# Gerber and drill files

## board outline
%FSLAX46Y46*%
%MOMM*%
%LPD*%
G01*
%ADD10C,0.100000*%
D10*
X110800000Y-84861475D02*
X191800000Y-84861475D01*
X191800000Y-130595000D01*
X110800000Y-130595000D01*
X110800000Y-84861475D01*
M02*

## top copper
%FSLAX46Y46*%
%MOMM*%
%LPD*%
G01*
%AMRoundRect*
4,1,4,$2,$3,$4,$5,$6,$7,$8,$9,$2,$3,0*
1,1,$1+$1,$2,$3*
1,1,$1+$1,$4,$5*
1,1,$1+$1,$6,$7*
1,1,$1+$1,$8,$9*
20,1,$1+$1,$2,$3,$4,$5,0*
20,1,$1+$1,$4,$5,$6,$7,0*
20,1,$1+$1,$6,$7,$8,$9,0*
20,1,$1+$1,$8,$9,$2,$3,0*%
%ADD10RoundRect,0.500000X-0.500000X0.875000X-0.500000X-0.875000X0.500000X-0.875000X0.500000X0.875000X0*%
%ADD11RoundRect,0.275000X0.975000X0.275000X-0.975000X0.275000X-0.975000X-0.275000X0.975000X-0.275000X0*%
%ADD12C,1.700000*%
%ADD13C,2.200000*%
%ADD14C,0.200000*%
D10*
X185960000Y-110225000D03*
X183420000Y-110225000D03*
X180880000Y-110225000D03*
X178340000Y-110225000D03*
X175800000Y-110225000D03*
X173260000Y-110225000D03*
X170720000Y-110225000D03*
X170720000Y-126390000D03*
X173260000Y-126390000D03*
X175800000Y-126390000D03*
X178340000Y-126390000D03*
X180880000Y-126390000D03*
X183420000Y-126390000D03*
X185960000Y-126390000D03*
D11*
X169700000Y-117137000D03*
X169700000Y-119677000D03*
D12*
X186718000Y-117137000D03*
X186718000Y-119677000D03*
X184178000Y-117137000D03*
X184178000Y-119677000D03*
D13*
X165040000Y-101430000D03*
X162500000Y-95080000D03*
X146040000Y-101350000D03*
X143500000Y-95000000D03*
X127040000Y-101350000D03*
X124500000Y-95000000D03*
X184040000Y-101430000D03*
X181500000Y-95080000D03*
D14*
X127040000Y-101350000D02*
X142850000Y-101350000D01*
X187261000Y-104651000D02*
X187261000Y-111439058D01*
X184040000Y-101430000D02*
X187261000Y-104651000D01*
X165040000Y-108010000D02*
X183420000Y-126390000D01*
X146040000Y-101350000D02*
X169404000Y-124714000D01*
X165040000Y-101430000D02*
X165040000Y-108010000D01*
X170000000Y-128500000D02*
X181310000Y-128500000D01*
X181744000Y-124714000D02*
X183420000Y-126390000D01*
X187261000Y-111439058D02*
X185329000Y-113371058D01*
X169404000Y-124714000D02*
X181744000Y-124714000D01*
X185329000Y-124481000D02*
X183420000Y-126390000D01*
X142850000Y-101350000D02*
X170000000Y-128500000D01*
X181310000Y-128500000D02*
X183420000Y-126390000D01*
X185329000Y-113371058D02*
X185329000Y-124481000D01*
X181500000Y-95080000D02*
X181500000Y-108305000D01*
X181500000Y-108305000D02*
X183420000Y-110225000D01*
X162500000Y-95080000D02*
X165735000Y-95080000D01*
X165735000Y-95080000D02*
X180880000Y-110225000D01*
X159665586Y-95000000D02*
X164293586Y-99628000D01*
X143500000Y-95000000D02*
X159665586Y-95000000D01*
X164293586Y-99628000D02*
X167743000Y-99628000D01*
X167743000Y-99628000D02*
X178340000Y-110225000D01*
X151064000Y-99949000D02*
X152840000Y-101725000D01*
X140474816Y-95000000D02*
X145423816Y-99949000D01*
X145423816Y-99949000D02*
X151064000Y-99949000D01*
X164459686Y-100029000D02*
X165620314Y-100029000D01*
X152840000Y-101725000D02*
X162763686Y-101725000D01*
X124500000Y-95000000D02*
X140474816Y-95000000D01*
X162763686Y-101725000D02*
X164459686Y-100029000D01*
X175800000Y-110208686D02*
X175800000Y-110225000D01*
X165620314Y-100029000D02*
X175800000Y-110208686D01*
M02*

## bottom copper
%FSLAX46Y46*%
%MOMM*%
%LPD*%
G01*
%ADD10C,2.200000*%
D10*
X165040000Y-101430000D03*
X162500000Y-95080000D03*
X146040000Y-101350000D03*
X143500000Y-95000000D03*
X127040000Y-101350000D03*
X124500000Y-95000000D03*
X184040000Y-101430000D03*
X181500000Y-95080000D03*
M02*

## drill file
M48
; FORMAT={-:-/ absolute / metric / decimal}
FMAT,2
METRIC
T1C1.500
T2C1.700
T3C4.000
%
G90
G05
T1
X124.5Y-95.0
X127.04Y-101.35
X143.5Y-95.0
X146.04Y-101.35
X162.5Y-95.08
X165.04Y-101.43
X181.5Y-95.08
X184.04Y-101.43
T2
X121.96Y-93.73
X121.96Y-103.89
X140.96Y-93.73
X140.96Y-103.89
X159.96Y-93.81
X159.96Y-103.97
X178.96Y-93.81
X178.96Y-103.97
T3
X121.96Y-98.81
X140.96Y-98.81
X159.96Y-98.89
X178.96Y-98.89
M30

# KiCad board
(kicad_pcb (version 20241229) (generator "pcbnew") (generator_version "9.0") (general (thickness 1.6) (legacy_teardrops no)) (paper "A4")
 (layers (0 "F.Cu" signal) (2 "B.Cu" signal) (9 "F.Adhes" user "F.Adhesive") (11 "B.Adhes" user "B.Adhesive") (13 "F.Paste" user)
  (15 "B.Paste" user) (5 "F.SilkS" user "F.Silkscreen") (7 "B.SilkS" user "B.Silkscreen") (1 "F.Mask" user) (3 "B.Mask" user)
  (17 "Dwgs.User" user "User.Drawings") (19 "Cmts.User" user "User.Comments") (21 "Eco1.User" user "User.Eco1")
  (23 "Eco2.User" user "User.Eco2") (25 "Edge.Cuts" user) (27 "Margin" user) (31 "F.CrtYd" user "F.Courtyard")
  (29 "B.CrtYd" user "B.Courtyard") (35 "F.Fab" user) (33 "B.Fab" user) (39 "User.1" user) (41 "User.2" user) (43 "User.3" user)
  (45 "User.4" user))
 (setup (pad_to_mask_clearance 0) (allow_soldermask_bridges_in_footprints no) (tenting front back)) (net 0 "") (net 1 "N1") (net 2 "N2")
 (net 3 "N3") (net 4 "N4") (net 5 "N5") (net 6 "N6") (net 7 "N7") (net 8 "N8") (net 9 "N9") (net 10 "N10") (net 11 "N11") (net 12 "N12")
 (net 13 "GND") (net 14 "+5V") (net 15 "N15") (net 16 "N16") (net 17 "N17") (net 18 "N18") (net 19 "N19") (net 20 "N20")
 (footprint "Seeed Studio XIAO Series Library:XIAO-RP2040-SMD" (layer "F.Cu") (at 178.34 118.225 -90)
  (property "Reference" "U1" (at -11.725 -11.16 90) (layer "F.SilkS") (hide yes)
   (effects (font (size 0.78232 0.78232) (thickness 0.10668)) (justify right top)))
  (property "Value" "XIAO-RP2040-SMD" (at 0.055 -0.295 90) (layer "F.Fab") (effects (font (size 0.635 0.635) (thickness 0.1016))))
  (pad "1" smd roundrect (at -8 -7.62 270) (size 2.75 2) (layers "F.Cu" "F.Mask" "F.Paste") (roundrect_rratio 0.25) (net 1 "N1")
   (solder_mask_margin 0.0508) (thermal_bridge_angle 45))
  (pad "2" smd roundrect (at -8 -5.08 270) (size 2.75 2) (layers "F.Cu" "F.Mask" "F.Paste") (roundrect_rratio 0.25) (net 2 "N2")
   (solder_mask_margin 0.0508) (thermal_bridge_angle 45))
  (pad "3" smd roundrect (at -8 -2.54 270) (size 2.75 2) (layers "F.Cu" "F.Mask" "F.Paste") (roundrect_rratio 0.25) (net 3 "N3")
   (solder_mask_margin 0.0508) (thermal_bridge_angle 45))
  (pad "4" smd roundrect (at -8 0 270) (size 2.75 2) (layers "F.Cu" "F.Mask" "F.Paste") (roundrect_rratio 0.25) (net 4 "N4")
   (solder_mask_margin 0.0508) (thermal_bridge_angle 45))
  (pad "5" smd roundrect (at -8 2.54 270) (size 2.75 2) (layers "F.Cu" "F.Mask" "F.Paste") (roundrect_rratio 0.25) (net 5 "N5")
   (solder_mask_margin 0.0508) (thermal_bridge_angle 45))
  (pad "6" smd roundrect (at -8 5.08 270) (size 2.75 2) (layers "F.Cu" "F.Mask" "F.Paste") (roundrect_rratio 0.25) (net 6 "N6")
   (solder_mask_margin 0.0508) (thermal_bridge_angle 45))
  (pad "7" smd roundrect (at -8 7.62 270) (size 2.75 2) (layers "F.Cu" "F.Mask" "F.Paste") (roundrect_rratio 0.25) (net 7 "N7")
   (solder_mask_margin 0.0508) (thermal_bridge_angle 45))
  (pad "8" smd roundrect (at 8.165 7.62 270) (size 2.75 2) (layers "F.Cu" "F.Mask" "F.Paste") (roundrect_rratio 0.25) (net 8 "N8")
   (solder_mask_margin 0.0508) (thermal_bridge_angle 45))
  (pad "9" smd roundrect (at 8.165 5.08 270) (size 2.75 2) (layers "F.Cu" "F.Mask" "F.Paste") (roundrect_rratio 0.25) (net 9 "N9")
   (solder_mask_margin 0.0508) (thermal_bridge_angle 45))
  (pad "10" smd roundrect (at 8.165 2.54 270) (size 2.75 2) (layers "F.Cu" "F.Mask" "F.Paste") (roundrect_rratio 0.25) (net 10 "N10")
   (solder_mask_margin 0.0508) (thermal_bridge_angle 45))
  (pad "11" smd roundrect (at 8.165 0 270) (size 2.75 2) (layers "F.Cu" "F.Mask" "F.Paste") (roundrect_rratio 0.25) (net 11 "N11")
   (solder_mask_margin 0.0508) (thermal_bridge_angle 45))
  (pad "12" smd roundrect (at 8.165 -2.54 270) (size 2.75 2) (layers "F.Cu" "F.Mask" "F.Paste") (roundrect_rratio 0.25) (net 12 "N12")
   (solder_mask_margin 0.0508) (thermal_bridge_angle 45))
  (pad "13" smd roundrect (at 8.165 -5.08 270) (size 2.75 2) (layers "F.Cu" "F.Mask" "F.Paste") (roundrect_rratio 0.25) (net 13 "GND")
   (solder_mask_margin 0.0508) (thermal_bridge_angle 45))
  (pad "14" smd roundrect (at 8.165 -7.62 270) (size 2.75 2) (layers "F.Cu" "F.Mask" "F.Paste") (roundrect_rratio 0.25) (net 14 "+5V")
   (solder_mask_margin 0.0508) (thermal_bridge_angle 45))
  (pad "15" smd roundrect (at -1.088 8.64 180) (size 2.5 1.1) (layers "F.Cu" "F.Mask" "F.Paste") (roundrect_rratio 0.25) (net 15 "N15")
   (thermal_bridge_angle 45))
  (pad "16" smd roundrect (at 1.452 8.64 180) (size 2.5 1.1) (layers "F.Cu" "F.Mask" "F.Paste") (roundrect_rratio 0.25) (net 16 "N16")
   (thermal_bridge_angle 45))
  (pad "17" smd circle (at -1.088 -8.378 270) (size 1.7 1.7) (layers "F.Cu" "F.Mask" "F.Paste") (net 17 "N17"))
  (pad "18" smd circle (at 1.452 -8.378 270) (size 1.7 1.7) (layers "F.Cu" "F.Mask" "F.Paste") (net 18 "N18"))
  (pad "19" smd circle (at -1.088 -5.838 270) (size 1.7 1.7) (layers "F.Cu" "F.Mask" "F.Paste") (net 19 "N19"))
  (pad "20" smd circle (at 1.452 -5.838 270) (size 1.7 1.7) (layers "F.Cu" "F.Mask" "F.Paste") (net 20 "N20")))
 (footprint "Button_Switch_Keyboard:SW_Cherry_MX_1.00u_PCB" (layer "F.Cu") (at 165.04 101.43 -90)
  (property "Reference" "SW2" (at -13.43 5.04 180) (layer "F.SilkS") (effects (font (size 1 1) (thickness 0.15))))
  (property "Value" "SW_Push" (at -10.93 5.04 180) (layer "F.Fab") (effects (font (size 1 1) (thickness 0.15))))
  (pad "" np_thru_hole circle (at -7.62 5.08 270) (size 1.7 1.7) (drill 1.7) (layers "*.Cu" "*.Mask"))
  (pad "" np_thru_hole circle (at -2.54 5.08 270) (size 4 4) (drill 4) (layers "*.Cu" "*.Mask"))
  (pad "" np_thru_hole circle (at 2.54 5.08 270) (size 1.7 1.7) (drill 1.7) (layers "*.Cu" "*.Mask"))
  (pad "1" thru_hole circle (at 0 0 270) (size 2.2 2.2) (drill 1.5) (layers "*.Cu" "*.Mask") (remove_unused_layers no) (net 13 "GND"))
  (pad "2" thru_hole circle (at -6.35 2.54 270) (size 2.2 2.2) (drill 1.5) (layers "*.Cu" "*.Mask") (remove_unused_layers no) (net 3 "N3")))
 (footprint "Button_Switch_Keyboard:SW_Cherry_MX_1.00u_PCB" (layer "F.Cu") (at 146.04 101.35 -90)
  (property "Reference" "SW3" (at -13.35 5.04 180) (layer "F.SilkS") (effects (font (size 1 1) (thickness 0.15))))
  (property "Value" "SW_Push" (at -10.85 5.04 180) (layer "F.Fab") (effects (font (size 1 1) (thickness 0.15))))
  (pad "" np_thru_hole circle (at -7.62 5.08 270) (size 1.7 1.7) (drill 1.7) (layers "*.Cu" "*.Mask"))
  (pad "" np_thru_hole circle (at -2.54 5.08 270) (size 4 4) (drill 4) (layers "*.Cu" "*.Mask"))
  (pad "" np_thru_hole circle (at 2.54 5.08 270) (size 1.7 1.7) (drill 1.7) (layers "*.Cu" "*.Mask"))
  (pad "1" thru_hole circle (at 0 0 270) (size 2.2 2.2) (drill 1.5) (layers "*.Cu" "*.Mask") (remove_unused_layers no) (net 13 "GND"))
  (pad "2" thru_hole circle (at -6.35 2.54 270) (size 2.2 2.2) (drill 1.5) (layers "*.Cu" "*.Mask") (remove_unused_layers no) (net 4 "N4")))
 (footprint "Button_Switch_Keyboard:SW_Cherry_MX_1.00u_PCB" (layer "F.Cu") (at 127.04 101.35 -90)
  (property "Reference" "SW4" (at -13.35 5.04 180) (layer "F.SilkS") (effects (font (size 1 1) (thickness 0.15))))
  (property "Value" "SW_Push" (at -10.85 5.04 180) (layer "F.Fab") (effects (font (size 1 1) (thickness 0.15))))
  (pad "" np_thru_hole circle (at -7.62 5.08 270) (size 1.7 1.7) (drill 1.7) (layers "*.Cu" "*.Mask"))
  (pad "" np_thru_hole circle (at -2.54 5.08 270) (size 4 4) (drill 4) (layers "*.Cu" "*.Mask"))
  (pad "" np_thru_hole circle (at 2.54 5.08 270) (size 1.7 1.7) (drill 1.7) (layers "*.Cu" "*.Mask"))
  (pad "1" thru_hole circle (at 0 0 270) (size 2.2 2.2) (drill 1.5) (layers "*.Cu" "*.Mask") (remove_unused_layers no) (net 13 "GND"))
  (pad "2" thru_hole circle (at -6.35 2.54 270) (size 2.2 2.2) (drill 1.5) (layers "*.Cu" "*.Mask") (remove_unused_layers no) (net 5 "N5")))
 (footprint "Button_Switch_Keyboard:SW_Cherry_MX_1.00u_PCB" (layer "F.Cu") (at 184.04 101.43 -90)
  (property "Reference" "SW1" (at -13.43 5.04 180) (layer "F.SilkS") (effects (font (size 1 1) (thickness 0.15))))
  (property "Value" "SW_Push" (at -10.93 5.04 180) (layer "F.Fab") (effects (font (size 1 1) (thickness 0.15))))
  (pad "" np_thru_hole circle (at -7.62 5.08 270) (size 1.7 1.7) (drill 1.7) (layers "*.Cu" "*.Mask"))
  (pad "" np_thru_hole circle (at -2.54 5.08 270) (size 4 4) (drill 4) (layers "*.Cu" "*.Mask"))
  (pad "" np_thru_hole circle (at 2.54 5.08 270) (size 1.7 1.7) (drill 1.7) (layers "*.Cu" "*.Mask"))
  (pad "1" thru_hole circle (at 0 0 270) (size 2.2 2.2) (drill 1.5) (layers "*.Cu" "*.Mask") (remove_unused_layers no) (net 13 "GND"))
  (pad "2" thru_hole circle (at -6.35 2.54 270) (size 2.2 2.2) (drill 1.5) (layers "*.Cu" "*.Mask") (remove_unused_layers no) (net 2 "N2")))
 (gr_rect (start 110.8 84.861475) (end 191.8 130.595) (stroke (width 0.1) (type solid)) (fill no) (layer "Edge.Cuts"))
 (segment (start 127.04 101.35) (end 142.85 101.35) (width 0.2) (layer "F.Cu") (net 13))
 (segment (start 187.261 104.651) (end 187.261 111.439058) (width 0.2) (layer "F.Cu") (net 13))
 (segment (start 184.04 101.43) (end 187.261 104.651) (width 0.2) (layer "F.Cu") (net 13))
 (segment (start 165.04 108.01) (end 183.42 126.39) (width 0.2) (layer "F.Cu") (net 13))
 (segment (start 146.04 101.35) (end 169.404 124.714) (width 0.2) (layer "F.Cu") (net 13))
 (segment (start 165.04 101.43) (end 165.04 108.01) (width 0.2) (layer "F.Cu") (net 13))
 (segment (start 170 128.5) (end 181.31 128.5) (width 0.2) (layer "F.Cu") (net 13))
 (segment (start 181.744 124.714) (end 183.42 126.39) (width 0.2) (layer "F.Cu") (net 13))
 (segment (start 187.261 111.439058) (end 185.329 113.371058) (width 0.2) (layer "F.Cu") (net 13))
 (segment (start 169.404 124.714) (end 181.744 124.714) (width 0.2) (layer "F.Cu") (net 13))
 (segment (start 185.329 124.481) (end 183.42 126.39) (width 0.2) (layer "F.Cu") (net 13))
 (segment (start 142.85 101.35) (end 170 128.5) (width 0.2) (layer "F.Cu") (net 13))
 (segment (start 181.31 128.5) (end 183.42 126.39) (width 0.2) (layer "F.Cu") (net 13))
 (segment (start 185.329 113.371058) (end 185.329 124.481) (width 0.2) (layer "F.Cu") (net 13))
 (segment (start 181.5 95.08) (end 181.5 108.305) (width 0.2) (layer "F.Cu") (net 2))
 (segment (start 181.5 108.305) (end 183.42 110.225) (width 0.2) (layer "F.Cu") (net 2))
 (segment (start 162.5 95.08) (end 165.735 95.08) (width 0.2) (layer "F.Cu") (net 3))
 (segment (start 165.735 95.08) (end 180.88 110.225) (width 0.2) (layer "F.Cu") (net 3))
 (segment (start 159.665586 95) (end 164.293586 99.628) (width 0.2) (layer "F.Cu") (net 4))
 (segment (start 143.5 95) (end 159.665586 95) (width 0.2) (layer "F.Cu") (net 4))
 (segment (start 164.293586 99.628) (end 167.743 99.628) (width 0.2) (layer "F.Cu") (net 4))
 (segment (start 167.743 99.628) (end 178.34 110.225) (width 0.2) (layer "F.Cu") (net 4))
 (segment (start 151.064 99.949) (end 152.84 101.725) (width 0.2) (layer "F.Cu") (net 5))
 (segment (start 140.474816 95) (end 145.423816 99.949) (width 0.2) (layer "F.Cu") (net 5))
 (segment (start 145.423816 99.949) (end 151.064 99.949) (width 0.2) (layer "F.Cu") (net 5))
 (segment (start 164.459686 100.029) (end 165.620314 100.029) (width 0.2) (layer "F.Cu") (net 5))
 (segment (start 152.84 101.725) (end 162.763686 101.725) (width 0.2) (layer "F.Cu") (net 5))
 (segment (start 124.5 95) (end 140.474816 95) (width 0.2) (layer "F.Cu") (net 5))
 (segment (start 162.763686 101.725) (end 164.459686 100.029) (width 0.2) (layer "F.Cu") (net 5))
 (segment (start 175.8 110.208686) (end 175.8 110.225) (width 0.2) (layer "F.Cu") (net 5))
 (segment (start 165.620314 100.029) (end 175.8 110.208686) (width 0.2) (layer "F.Cu") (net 5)))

